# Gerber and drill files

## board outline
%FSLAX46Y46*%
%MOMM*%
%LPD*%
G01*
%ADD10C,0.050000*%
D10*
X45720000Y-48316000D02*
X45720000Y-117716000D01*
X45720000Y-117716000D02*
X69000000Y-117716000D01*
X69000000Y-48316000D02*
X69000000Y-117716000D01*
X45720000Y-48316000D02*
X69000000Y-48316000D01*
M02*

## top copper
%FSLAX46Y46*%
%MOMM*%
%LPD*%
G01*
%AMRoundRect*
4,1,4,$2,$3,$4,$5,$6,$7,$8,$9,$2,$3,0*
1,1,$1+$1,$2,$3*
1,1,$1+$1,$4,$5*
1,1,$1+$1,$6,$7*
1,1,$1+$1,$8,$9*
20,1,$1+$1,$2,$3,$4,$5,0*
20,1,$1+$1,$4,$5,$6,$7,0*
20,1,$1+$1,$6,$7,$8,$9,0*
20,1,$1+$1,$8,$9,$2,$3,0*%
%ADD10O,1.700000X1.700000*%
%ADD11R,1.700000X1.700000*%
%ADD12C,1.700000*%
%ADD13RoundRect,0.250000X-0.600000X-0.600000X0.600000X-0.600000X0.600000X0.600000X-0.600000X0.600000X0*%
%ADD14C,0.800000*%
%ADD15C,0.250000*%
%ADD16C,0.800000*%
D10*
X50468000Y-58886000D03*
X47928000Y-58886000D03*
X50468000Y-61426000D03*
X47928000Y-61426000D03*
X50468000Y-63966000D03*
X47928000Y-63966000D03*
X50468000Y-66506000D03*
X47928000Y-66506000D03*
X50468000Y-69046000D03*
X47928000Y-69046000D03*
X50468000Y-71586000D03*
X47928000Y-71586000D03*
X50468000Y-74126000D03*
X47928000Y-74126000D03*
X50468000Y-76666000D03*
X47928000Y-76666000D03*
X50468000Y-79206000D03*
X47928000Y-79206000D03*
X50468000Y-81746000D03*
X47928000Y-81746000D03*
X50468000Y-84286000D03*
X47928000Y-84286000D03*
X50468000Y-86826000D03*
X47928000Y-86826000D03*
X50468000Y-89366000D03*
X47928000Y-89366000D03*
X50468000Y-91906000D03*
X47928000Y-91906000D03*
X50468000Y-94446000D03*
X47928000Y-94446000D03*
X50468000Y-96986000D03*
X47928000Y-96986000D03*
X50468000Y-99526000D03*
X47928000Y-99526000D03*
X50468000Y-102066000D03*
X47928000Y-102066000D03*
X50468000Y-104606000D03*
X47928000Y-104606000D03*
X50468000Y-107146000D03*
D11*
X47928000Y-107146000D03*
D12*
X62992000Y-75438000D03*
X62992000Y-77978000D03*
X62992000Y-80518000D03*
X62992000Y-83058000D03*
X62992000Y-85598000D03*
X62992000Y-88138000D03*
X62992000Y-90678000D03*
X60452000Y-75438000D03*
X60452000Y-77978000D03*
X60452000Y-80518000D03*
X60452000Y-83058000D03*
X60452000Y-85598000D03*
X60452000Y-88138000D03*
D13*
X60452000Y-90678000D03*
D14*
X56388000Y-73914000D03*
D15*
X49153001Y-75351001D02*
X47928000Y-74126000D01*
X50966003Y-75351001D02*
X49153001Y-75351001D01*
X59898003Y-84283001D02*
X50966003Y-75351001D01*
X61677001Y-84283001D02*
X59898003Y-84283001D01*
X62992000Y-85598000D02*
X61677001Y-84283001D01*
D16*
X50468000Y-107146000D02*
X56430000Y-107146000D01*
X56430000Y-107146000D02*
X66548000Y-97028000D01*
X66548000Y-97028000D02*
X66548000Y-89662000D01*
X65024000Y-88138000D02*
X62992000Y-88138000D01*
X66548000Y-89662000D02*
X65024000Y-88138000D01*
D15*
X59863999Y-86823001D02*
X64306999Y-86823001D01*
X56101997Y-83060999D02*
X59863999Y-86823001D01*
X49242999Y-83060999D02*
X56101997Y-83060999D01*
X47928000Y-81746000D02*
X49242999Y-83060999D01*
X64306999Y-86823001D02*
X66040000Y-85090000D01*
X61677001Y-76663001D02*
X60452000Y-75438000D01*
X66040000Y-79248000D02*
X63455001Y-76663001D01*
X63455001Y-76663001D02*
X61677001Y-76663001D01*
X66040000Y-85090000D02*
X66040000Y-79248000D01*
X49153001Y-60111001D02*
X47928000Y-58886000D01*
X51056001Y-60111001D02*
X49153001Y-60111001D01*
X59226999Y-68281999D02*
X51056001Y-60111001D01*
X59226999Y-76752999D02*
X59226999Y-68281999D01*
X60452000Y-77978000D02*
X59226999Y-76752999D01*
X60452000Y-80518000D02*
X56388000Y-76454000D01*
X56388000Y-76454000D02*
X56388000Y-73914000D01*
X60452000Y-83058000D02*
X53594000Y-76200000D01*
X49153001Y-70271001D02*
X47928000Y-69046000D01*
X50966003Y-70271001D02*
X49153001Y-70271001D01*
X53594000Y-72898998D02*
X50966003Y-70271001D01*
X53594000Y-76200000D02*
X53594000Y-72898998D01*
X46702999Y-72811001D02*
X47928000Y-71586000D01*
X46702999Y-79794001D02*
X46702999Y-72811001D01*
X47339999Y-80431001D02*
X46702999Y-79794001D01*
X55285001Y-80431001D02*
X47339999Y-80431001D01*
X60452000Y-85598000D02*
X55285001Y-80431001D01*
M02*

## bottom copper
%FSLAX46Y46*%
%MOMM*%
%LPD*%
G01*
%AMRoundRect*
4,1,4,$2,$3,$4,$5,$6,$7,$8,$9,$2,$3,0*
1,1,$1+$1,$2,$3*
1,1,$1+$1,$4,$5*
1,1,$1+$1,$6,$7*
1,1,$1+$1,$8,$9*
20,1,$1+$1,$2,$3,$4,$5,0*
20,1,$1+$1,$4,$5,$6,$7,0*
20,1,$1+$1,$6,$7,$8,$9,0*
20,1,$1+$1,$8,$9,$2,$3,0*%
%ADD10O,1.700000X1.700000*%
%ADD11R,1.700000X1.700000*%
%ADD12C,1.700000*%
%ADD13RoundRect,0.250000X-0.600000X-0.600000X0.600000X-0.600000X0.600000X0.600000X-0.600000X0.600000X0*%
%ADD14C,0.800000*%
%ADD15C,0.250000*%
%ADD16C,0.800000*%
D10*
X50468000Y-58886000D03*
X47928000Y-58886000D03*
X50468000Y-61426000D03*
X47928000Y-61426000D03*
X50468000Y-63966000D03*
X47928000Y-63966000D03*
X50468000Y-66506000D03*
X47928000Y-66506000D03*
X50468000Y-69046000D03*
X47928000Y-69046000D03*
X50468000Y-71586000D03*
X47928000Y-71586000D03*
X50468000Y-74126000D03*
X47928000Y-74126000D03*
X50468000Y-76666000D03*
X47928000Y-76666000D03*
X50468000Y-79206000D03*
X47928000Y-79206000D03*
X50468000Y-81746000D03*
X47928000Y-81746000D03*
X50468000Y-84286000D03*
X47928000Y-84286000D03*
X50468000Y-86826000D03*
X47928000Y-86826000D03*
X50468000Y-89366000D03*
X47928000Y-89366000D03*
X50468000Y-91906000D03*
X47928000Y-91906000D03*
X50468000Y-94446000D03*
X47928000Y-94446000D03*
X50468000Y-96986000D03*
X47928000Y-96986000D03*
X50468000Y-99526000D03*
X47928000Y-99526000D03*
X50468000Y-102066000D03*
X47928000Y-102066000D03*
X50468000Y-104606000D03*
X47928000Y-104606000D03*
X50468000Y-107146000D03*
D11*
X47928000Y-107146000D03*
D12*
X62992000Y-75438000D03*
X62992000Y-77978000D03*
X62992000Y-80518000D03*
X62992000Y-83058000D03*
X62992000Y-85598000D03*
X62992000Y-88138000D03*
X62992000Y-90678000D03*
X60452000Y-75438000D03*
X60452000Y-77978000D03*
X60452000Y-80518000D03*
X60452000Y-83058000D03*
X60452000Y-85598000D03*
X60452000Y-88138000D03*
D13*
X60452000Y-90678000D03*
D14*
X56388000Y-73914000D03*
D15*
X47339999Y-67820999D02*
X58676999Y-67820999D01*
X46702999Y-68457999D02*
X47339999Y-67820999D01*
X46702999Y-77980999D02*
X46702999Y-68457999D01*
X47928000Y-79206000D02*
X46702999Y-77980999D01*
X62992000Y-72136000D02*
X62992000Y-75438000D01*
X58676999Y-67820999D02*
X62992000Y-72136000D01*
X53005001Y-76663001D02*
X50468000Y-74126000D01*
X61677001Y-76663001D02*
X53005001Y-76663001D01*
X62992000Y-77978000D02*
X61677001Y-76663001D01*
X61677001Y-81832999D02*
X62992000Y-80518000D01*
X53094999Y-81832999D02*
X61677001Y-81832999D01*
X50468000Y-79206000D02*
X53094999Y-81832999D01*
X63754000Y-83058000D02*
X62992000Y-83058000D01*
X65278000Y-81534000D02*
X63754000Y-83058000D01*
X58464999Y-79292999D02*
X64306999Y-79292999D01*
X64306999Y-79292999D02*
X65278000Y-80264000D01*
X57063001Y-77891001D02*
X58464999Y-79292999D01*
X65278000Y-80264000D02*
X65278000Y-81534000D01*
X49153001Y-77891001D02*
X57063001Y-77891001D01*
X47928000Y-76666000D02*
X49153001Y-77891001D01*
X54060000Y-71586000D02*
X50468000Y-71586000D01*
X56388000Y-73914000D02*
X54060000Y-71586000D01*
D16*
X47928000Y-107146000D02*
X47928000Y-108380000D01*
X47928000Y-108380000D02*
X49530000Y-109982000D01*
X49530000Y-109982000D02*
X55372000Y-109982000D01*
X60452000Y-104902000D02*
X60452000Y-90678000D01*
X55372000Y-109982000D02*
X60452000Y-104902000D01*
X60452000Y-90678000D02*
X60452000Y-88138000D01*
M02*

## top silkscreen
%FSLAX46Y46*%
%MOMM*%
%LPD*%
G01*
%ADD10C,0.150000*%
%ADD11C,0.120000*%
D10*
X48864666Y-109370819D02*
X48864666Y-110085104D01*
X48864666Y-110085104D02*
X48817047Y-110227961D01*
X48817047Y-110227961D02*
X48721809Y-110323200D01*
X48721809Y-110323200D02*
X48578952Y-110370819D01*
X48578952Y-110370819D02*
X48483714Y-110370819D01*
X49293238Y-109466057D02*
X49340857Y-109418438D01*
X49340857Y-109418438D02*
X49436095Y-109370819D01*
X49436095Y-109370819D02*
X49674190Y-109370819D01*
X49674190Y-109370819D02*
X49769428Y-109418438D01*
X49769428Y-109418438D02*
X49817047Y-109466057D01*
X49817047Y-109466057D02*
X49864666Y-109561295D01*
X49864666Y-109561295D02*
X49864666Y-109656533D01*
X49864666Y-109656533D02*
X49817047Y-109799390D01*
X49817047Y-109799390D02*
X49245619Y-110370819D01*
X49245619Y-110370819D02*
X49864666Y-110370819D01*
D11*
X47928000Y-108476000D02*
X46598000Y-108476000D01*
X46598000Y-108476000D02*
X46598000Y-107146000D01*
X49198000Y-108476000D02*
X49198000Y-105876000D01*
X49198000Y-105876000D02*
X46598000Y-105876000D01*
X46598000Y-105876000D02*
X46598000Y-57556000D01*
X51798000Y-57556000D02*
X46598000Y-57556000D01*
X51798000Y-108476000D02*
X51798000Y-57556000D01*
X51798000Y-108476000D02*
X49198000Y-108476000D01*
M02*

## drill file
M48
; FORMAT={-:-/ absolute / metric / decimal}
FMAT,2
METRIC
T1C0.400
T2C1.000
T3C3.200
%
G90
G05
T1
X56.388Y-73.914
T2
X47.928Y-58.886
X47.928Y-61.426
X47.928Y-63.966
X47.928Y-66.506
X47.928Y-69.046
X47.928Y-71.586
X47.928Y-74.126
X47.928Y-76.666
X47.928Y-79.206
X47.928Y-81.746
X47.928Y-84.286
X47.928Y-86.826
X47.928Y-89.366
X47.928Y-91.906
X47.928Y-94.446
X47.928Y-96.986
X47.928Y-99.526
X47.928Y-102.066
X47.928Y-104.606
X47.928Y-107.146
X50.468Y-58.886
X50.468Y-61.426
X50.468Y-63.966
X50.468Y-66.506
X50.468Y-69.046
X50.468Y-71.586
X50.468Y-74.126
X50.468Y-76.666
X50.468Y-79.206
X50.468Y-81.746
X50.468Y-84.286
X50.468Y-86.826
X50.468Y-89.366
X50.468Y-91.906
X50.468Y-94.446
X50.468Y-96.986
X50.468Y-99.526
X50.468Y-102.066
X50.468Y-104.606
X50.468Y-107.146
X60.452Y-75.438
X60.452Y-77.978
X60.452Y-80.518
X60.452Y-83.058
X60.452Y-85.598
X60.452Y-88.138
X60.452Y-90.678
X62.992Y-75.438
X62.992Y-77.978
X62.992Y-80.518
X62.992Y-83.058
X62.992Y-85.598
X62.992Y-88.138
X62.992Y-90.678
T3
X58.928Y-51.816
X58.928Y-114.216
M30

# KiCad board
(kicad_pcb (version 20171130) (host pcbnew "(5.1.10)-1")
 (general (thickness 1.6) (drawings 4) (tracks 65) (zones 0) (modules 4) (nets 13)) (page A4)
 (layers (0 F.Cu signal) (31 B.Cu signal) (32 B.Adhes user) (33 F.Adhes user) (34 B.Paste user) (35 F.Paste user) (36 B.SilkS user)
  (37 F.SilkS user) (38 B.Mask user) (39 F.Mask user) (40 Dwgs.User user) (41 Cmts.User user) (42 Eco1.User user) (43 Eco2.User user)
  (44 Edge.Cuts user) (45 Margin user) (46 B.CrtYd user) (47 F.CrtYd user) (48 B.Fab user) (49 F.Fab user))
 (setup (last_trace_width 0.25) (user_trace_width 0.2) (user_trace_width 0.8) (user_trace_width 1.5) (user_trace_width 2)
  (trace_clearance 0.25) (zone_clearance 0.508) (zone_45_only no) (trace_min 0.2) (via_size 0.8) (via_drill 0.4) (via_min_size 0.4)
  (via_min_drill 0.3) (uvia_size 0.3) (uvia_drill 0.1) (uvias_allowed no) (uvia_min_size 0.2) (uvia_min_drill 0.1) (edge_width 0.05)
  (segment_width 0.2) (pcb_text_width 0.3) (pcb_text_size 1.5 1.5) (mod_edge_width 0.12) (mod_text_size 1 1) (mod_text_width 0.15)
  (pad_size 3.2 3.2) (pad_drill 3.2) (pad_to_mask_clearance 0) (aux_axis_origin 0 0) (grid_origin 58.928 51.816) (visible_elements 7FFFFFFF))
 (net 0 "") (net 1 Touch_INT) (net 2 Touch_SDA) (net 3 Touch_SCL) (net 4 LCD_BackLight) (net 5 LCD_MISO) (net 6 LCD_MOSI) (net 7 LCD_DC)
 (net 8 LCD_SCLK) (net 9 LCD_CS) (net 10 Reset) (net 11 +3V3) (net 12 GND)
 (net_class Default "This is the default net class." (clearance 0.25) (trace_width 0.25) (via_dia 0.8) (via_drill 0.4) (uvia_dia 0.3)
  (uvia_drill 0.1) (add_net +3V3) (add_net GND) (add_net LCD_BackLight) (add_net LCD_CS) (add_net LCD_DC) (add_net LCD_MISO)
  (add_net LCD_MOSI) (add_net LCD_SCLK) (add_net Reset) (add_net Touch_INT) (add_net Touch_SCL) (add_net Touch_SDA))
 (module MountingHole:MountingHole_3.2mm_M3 (layer F.Cu) (at 58.928 114.216)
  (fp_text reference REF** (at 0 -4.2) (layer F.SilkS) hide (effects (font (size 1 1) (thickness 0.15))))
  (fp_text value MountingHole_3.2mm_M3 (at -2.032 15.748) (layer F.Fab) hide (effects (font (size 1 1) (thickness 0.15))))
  (pad 1 np_thru_hole circle (at 0 0) (size 3.2 3.2) (drill 3.2) (layers *.Cu *.Mask)))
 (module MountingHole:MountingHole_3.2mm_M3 (layer F.Cu) (at 58.928 51.816)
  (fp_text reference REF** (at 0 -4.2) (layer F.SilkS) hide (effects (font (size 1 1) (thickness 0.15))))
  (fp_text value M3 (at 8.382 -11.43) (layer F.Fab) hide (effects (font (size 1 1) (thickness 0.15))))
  (pad 1 np_thru_hole circle (at 0 0) (size 3.2 3.2) (drill 3.2) (layers *.Cu *.Mask)))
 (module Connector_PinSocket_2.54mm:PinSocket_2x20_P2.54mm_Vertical (layer F.Cu) (at 47.928 107.146 180)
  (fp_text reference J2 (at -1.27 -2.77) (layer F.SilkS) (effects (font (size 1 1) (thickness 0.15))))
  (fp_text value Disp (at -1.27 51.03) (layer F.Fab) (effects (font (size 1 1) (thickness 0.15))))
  (fp_line (start 0 -1.33) (end 1.33 -1.33) (layer F.SilkS) (width 0.12))
  (fp_line (start 1.33 -1.33) (end 1.33 0) (layer F.SilkS) (width 0.12))
  (fp_line (start -1.27 -1.33) (end -1.27 1.27) (layer F.SilkS) (width 0.12))
  (fp_line (start -1.27 1.27) (end 1.33 1.27) (layer F.SilkS) (width 0.12))
  (fp_line (start 1.33 1.27) (end 1.33 49.59) (layer F.SilkS) (width 0.12))
  (fp_line (start -3.87 49.59) (end 1.33 49.59) (layer F.SilkS) (width 0.12))
  (fp_line (start -3.87 -1.33) (end -3.87 49.59) (layer F.SilkS) (width 0.12))
  (fp_line (start -3.87 -1.33) (end -1.27 -1.33) (layer F.SilkS) (width 0.12))
  (pad 40 thru_hole oval (at -2.54 48.26 180) (size 1.7 1.7) (drill 1) (layers *.Cu *.Mask))
  (pad 39 thru_hole oval (at 0 48.26 180) (size 1.7 1.7) (drill 1) (layers *.Cu *.Mask) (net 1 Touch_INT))
  (pad 38 thru_hole oval (at -2.54 45.72 180) (size 1.7 1.7) (drill 1) (layers *.Cu *.Mask))
  (pad 37 thru_hole oval (at 0 45.72 180) (size 1.7 1.7) (drill 1) (layers *.Cu *.Mask))
  (pad 36 thru_hole oval (at -2.54 43.18 180) (size 1.7 1.7) (drill 1) (layers *.Cu *.Mask))
  (pad 35 thru_hole oval (at 0 43.18 180) (size 1.7 1.7) (drill 1) (layers *.Cu *.Mask))
  (pad 34 thru_hole oval (at -2.54 40.64 180) (size 1.7 1.7) (drill 1) (layers *.Cu *.Mask))
  (pad 33 thru_hole oval (at 0 40.64 180) (size 1.7 1.7) (drill 1) (layers *.Cu *.Mask))
  (pad 32 thru_hole oval (at -2.54 38.1 180) (size 1.7 1.7) (drill 1) (layers *.Cu *.Mask))
  (pad 31 thru_hole oval (at 0 38.1 180) (size 1.7 1.7) (drill 1) (layers *.Cu *.Mask) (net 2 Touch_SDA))
  (pad 30 thru_hole oval (at -2.54 35.56 180) (size 1.7 1.7) (drill 1) (layers *.Cu *.Mask) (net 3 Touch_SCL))
  (pad 29 thru_hole oval (at 0 35.56 180) (size 1.7 1.7) (drill 1) (layers *.Cu *.Mask) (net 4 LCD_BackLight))
  (pad 28 thru_hole oval (at -2.54 33.02 180) (size 1.7 1.7) (drill 1) (layers *.Cu *.Mask) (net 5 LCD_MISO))
  (pad 27 thru_hole oval (at 0 33.02 180) (size 1.7 1.7) (drill 1) (layers *.Cu *.Mask) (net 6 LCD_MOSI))
  (pad 26 thru_hole oval (at -2.54 30.48 180) (size 1.7 1.7) (drill 1) (layers *.Cu *.Mask))
  (pad 25 thru_hole oval (at 0 30.48 180) (size 1.7 1.7) (drill 1) (layers *.Cu *.Mask) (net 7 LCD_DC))
  (pad 24 thru_hole oval (at -2.54 27.94 180) (size 1.7 1.7) (drill 1) (layers *.Cu *.Mask) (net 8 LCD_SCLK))
  (pad 23 thru_hole oval (at 0 27.94 180) (size 1.7 1.7) (drill 1) (layers *.Cu *.Mask) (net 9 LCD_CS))
  (pad 22 thru_hole oval (at -2.54 25.4 180) (size 1.7 1.7) (drill 1) (layers *.Cu *.Mask))
  (pad 21 thru_hole oval (at 0 25.4 180) (size 1.7 1.7) (drill 1) (layers *.Cu *.Mask) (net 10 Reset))
  (pad 20 thru_hole oval (at -2.54 22.86 180) (size 1.7 1.7) (drill 1) (layers *.Cu *.Mask))
  (pad 19 thru_hole oval (at 0 22.86 180) (size 1.7 1.7) (drill 1) (layers *.Cu *.Mask))
  (pad 18 thru_hole oval (at -2.54 20.32 180) (size 1.7 1.7) (drill 1) (layers *.Cu *.Mask))
  (pad 17 thru_hole oval (at 0 20.32 180) (size 1.7 1.7) (drill 1) (layers *.Cu *.Mask))
  (pad 16 thru_hole oval (at -2.54 17.78 180) (size 1.7 1.7) (drill 1) (layers *.Cu *.Mask))
  (pad 15 thru_hole oval (at 0 17.78 180) (size 1.7 1.7) (drill 1) (layers *.Cu *.Mask))
  (pad 14 thru_hole oval (at -2.54 15.24 180) (size 1.7 1.7) (drill 1) (layers *.Cu *.Mask))
  (pad 13 thru_hole oval (at 0 15.24 180) (size 1.7 1.7) (drill 1) (layers *.Cu *.Mask))
  (pad 12 thru_hole oval (at -2.54 12.7 180) (size 1.7 1.7) (drill 1) (layers *.Cu *.Mask))
  (pad 11 thru_hole oval (at 0 12.7 180) (size 1.7 1.7) (drill 1) (layers *.Cu *.Mask))
  (pad 10 thru_hole oval (at -2.54 10.16 180) (size 1.7 1.7) (drill 1) (layers *.Cu *.Mask))
  (pad 9 thru_hole oval (at 0 10.16 180) (size 1.7 1.7) (drill 1) (layers *.Cu *.Mask))
  (pad 8 thru_hole oval (at -2.54 7.62 180) (size 1.7 1.7) (drill 1) (layers *.Cu *.Mask))
  (pad 7 thru_hole oval (at 0 7.62 180) (size 1.7 1.7) (drill 1) (layers *.Cu *.Mask))
  (pad 6 thru_hole oval (at -2.54 5.08 180) (size 1.7 1.7) (drill 1) (layers *.Cu *.Mask))
  (pad 5 thru_hole oval (at 0 5.08 180) (size 1.7 1.7) (drill 1) (layers *.Cu *.Mask))
  (pad 4 thru_hole oval (at -2.54 2.54 180) (size 1.7 1.7) (drill 1) (layers *.Cu *.Mask))
  (pad 3 thru_hole oval (at 0 2.54 180) (size 1.7 1.7) (drill 1) (layers *.Cu *.Mask))
  (pad 2 thru_hole oval (at -2.54 0 180) (size 1.7 1.7) (drill 1) (layers *.Cu *.Mask) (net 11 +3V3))
  (pad 1 thru_hole rect (at 0 0 180) (size 1.7 1.7) (drill 1) (layers *.Cu *.Mask) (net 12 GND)))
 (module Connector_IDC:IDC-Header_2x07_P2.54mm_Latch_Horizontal (layer B.Cu) (at 60.452 90.678)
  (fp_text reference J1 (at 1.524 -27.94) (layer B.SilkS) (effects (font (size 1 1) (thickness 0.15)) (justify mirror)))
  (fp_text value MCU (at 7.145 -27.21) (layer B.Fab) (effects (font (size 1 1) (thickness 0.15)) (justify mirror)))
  (pad 14 thru_hole circle (at 2.54 -15.24) (size 1.7 1.7) (drill 1) (layers *.Cu *.Mask) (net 9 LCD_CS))
  (pad 12 thru_hole circle (at 2.54 -12.7) (size 1.7 1.7) (drill 1) (layers *.Cu *.Mask) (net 5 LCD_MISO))
  (pad 10 thru_hole circle (at 2.54 -10.16) (size 1.7 1.7) (drill 1) (layers *.Cu *.Mask) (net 8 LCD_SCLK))
  (pad 8 thru_hole circle (at 2.54 -7.62) (size 1.7 1.7) (drill 1) (layers *.Cu *.Mask) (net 7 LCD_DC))
  (pad 6 thru_hole circle (at 2.54 -5.08) (size 1.7 1.7) (drill 1) (layers *.Cu *.Mask) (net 6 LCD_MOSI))
  (pad 4 thru_hole circle (at 2.54 -2.54) (size 1.7 1.7) (drill 1) (layers *.Cu *.Mask) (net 11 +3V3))
  (pad 2 thru_hole circle (at 2.54 0) (size 1.7 1.7) (drill 1) (layers *.Cu *.Mask))
  (pad 13 thru_hole circle (at 0 -15.24) (size 1.7 1.7) (drill 1) (layers *.Cu *.Mask) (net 10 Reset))
  (pad 11 thru_hole circle (at 0 -12.7) (size 1.7 1.7) (drill 1) (layers *.Cu *.Mask) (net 1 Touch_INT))
  (pad 9 thru_hole circle (at 0 -10.16) (size 1.7 1.7) (drill 1) (layers *.Cu *.Mask) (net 3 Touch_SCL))
  (pad 7 thru_hole circle (at 0 -7.62) (size 1.7 1.7) (drill 1) (layers *.Cu *.Mask) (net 2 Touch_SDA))
  (pad 5 thru_hole circle (at 0 -5.08) (size 1.7 1.7) (drill 1) (layers *.Cu *.Mask) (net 4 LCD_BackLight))
  (pad 3 thru_hole circle (at 0 -2.54) (size 1.7 1.7) (drill 1) (layers *.Cu *.Mask) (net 12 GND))
  (pad 1 thru_hole roundrect (at 0 0) (size 1.7 1.7) (drill 1) (layers *.Cu *.Mask) (roundrect_rratio 0.147059) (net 12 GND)))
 (gr_line (start 45.72 48.316) (end 45.72 117.716) (layer Edge.Cuts) (width 0.05))
 (gr_line (start 45.72 117.716) (end 69 117.716) (layer Edge.Cuts) (width 0.05))
 (gr_line (start 69 48.316) (end 69 117.716) (layer Edge.Cuts) (width 0.05))
 (gr_line (start 45.72 48.316) (end 69 48.316) (layer Edge.Cuts) (width 0.05))
 (segment (start 47.339999 67.820999) (end 58.676999 67.820999) (width 0.25) (layer B.Cu) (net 9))
 (segment (start 46.702999 68.457999) (end 47.339999 67.820999) (width 0.25) (layer B.Cu) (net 9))
 (segment (start 46.702999 77.980999) (end 46.702999 68.457999) (width 0.25) (layer B.Cu) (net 9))
 (segment (start 47.928 79.206) (end 46.702999 77.980999) (width 0.25) (layer B.Cu) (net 9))
 (segment (start 62.992 72.136) (end 62.992 75.438) (width 0.25) (layer B.Cu) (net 9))
 (segment (start 58.676999 67.820999) (end 62.992 72.136) (width 0.25) (layer B.Cu) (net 9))
 (segment (start 53.005001 76.663001) (end 50.468 74.126) (width 0.25) (layer B.Cu) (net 5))
 (segment (start 61.677001 76.663001) (end 53.005001 76.663001) (width 0.25) (layer B.Cu) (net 5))
 (segment (start 62.992 77.978) (end 61.677001 76.663001) (width 0.25) (layer B.Cu) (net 5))
 (segment (start 61.677001 81.832999) (end 62.992 80.518) (width 0.25) (layer B.Cu) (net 8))
 (segment (start 53.094999 81.832999) (end 61.677001 81.832999) (width 0.25) (layer B.Cu) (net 8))
 (segment (start 50.468 79.206) (end 53.094999 81.832999) (width 0.25) (layer B.Cu) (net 8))
 (segment (start 63.754 83.058) (end 62.992 83.058) (width 0.25) (layer B.Cu) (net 7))
 (segment (start 65.278 81.534) (end 63.754 83.058) (width 0.25) (layer B.Cu) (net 7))
 (segment (start 58.464999 79.292999) (end 64.306999 79.292999) (width 0.25) (layer B.Cu) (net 7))
 (segment (start 64.306999 79.292999) (end 65.278 80.264) (width 0.25) (layer B.Cu) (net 7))
 (segment (start 57.063001 77.891001) (end 58.464999 79.292999) (width 0.25) (layer B.Cu) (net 7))
 (segment (start 65.278 80.264) (end 65.278 81.534) (width 0.25) (layer B.Cu) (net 7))
 (segment (start 49.153001 77.891001) (end 57.063001 77.891001) (width 0.25) (layer B.Cu) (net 7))
 (segment (start 47.928 76.666) (end 49.153001 77.891001) (width 0.25) (layer B.Cu) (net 7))
 (segment (start 49.153001 75.351001) (end 47.928 74.126) (width 0.25) (layer F.Cu) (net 6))
 (segment (start 50.966003 75.351001) (end 49.153001 75.351001) (width 0.25) (layer F.Cu) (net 6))
 (segment (start 59.898003 84.283001) (end 50.966003 75.351001) (width 0.25) (layer F.Cu) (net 6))
 (segment (start 61.677001 84.283001) (end 59.898003 84.283001) (width 0.25) (layer F.Cu) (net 6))
 (segment (start 62.992 85.598) (end 61.677001 84.283001) (width 0.25) (layer F.Cu) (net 6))
 (segment (start 50.468 107.146) (end 56.43 107.146) (width 0.8) (layer F.Cu) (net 11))
 (segment (start 56.43 107.146) (end 66.548 97.028) (width 0.8) (layer F.Cu) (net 11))
 (segment (start 66.548 97.028) (end 66.548 89.662) (width 0.8) (layer F.Cu) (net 11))
 (segment (start 65.024 88.138) (end 62.992 88.138) (width 0.8) (layer F.Cu) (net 11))
 (segment (start 66.548 89.662) (end 65.024 88.138) (width 0.8) (layer F.Cu) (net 11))
 (segment (start 59.863999 86.823001) (end 64.306999 86.823001) (width 0.25) (layer F.Cu) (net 10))
 (segment (start 56.101997 83.060999) (end 59.863999 86.823001) (width 0.25) (layer F.Cu) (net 10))
 (segment (start 49.242999 83.060999) (end 56.101997 83.060999) (width 0.25) (layer F.Cu) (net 10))
 (segment (start 47.928 81.746) (end 49.242999 83.060999) (width 0.25) (layer F.Cu) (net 10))
 (segment (start 64.306999 86.823001) (end 66.04 85.09) (width 0.25) (layer F.Cu) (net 10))
 (segment (start 61.677001 76.663001) (end 60.452 75.438) (width 0.25) (layer F.Cu) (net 10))
 (segment (start 66.04 79.248) (end 63.455001 76.663001) (width 0.25) (layer F.Cu) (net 10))
 (segment (start 63.455001 76.663001) (end 61.677001 76.663001) (width 0.25) (layer F.Cu) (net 10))
 (segment (start 66.04 85.09) (end 66.04 79.248) (width 0.25) (layer F.Cu) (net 10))
 (segment (start 49.153001 60.111001) (end 47.928 58.886) (width 0.25) (layer F.Cu) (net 1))
 (segment (start 51.056001 60.111001) (end 49.153001 60.111001) (width 0.25) (layer F.Cu) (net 1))
 (segment (start 59.226999 68.281999) (end 51.056001 60.111001) (width 0.25) (layer F.Cu) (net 1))
 (segment (start 59.226999 76.752999) (end 59.226999 68.281999) (width 0.25) (layer F.Cu) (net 1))
 (segment (start 60.452 77.978) (end 59.226999 76.752999) (width 0.25) (layer F.Cu) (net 1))
 (segment (start 60.452 80.518) (end 56.388 76.454) (width 0.25) (layer F.Cu) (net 3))
 (via (at 56.388 73.914) (size 0.8) (drill 0.4) (layers F.Cu B.Cu) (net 3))
 (segment (start 56.388 76.454) (end 56.388 73.914) (width 0.25) (layer F.Cu) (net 3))
 (segment (start 54.06 71.586) (end 50.468 71.586) (width 0.25) (layer B.Cu) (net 3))
 (segment (start 56.388 73.914) (end 54.06 71.586) (width 0.25) (layer B.Cu) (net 3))
 (segment (start 60.452 83.058) (end 53.594 76.2) (width 0.25) (layer F.Cu) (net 2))
 (segment (start 49.153001 70.271001) (end 47.928 69.046) (width 0.25) (layer F.Cu) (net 2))
 (segment (start 50.966003 70.271001) (end 49.153001 70.271001) (width 0.25) (layer F.Cu) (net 2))
 (segment (start 53.594 72.898998) (end 50.966003 70.271001) (width 0.25) (layer F.Cu) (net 2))
 (segment (start 53.594 76.2) (end 53.594 72.898998) (width 0.25) (layer F.Cu) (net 2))
 (segment (start 46.702999 72.811001) (end 47.928 71.586) (width 0.25) (layer F.Cu) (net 4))
 (segment (start 46.702999 79.794001) (end 46.702999 72.811001) (width 0.25) (layer F.Cu) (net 4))
 (segment (start 47.339999 80.431001) (end 46.702999 79.794001) (width 0.25) (layer F.Cu) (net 4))
 (segment (start 55.285001 80.431001) (end 47.339999 80.431001) (width 0.25) (layer F.Cu) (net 4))
 (segment (start 60.452 85.598) (end 55.285001 80.431001) (width 0.25) (layer F.Cu) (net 4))
 (segment (start 47.928 107.146) (end 47.928 108.38) (width 0.8) (layer B.Cu) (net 12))
 (segment (start 47.928 108.38) (end 49.53 109.982) (width 0.8) (layer B.Cu) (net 12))
 (segment (start 49.53 109.982) (end 55.372 109.982) (width 0.8) (layer B.Cu) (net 12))
 (segment (start 60.452 104.902) (end 60.452 90.678) (width 0.8) (layer B.Cu) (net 12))
 (segment (start 55.372 109.982) (end 60.452 104.902) (width 0.8) (layer B.Cu) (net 12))
 (segment (start 60.452 90.678) (end 60.452 88.138) (width 0.8) (layer B.Cu) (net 12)))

